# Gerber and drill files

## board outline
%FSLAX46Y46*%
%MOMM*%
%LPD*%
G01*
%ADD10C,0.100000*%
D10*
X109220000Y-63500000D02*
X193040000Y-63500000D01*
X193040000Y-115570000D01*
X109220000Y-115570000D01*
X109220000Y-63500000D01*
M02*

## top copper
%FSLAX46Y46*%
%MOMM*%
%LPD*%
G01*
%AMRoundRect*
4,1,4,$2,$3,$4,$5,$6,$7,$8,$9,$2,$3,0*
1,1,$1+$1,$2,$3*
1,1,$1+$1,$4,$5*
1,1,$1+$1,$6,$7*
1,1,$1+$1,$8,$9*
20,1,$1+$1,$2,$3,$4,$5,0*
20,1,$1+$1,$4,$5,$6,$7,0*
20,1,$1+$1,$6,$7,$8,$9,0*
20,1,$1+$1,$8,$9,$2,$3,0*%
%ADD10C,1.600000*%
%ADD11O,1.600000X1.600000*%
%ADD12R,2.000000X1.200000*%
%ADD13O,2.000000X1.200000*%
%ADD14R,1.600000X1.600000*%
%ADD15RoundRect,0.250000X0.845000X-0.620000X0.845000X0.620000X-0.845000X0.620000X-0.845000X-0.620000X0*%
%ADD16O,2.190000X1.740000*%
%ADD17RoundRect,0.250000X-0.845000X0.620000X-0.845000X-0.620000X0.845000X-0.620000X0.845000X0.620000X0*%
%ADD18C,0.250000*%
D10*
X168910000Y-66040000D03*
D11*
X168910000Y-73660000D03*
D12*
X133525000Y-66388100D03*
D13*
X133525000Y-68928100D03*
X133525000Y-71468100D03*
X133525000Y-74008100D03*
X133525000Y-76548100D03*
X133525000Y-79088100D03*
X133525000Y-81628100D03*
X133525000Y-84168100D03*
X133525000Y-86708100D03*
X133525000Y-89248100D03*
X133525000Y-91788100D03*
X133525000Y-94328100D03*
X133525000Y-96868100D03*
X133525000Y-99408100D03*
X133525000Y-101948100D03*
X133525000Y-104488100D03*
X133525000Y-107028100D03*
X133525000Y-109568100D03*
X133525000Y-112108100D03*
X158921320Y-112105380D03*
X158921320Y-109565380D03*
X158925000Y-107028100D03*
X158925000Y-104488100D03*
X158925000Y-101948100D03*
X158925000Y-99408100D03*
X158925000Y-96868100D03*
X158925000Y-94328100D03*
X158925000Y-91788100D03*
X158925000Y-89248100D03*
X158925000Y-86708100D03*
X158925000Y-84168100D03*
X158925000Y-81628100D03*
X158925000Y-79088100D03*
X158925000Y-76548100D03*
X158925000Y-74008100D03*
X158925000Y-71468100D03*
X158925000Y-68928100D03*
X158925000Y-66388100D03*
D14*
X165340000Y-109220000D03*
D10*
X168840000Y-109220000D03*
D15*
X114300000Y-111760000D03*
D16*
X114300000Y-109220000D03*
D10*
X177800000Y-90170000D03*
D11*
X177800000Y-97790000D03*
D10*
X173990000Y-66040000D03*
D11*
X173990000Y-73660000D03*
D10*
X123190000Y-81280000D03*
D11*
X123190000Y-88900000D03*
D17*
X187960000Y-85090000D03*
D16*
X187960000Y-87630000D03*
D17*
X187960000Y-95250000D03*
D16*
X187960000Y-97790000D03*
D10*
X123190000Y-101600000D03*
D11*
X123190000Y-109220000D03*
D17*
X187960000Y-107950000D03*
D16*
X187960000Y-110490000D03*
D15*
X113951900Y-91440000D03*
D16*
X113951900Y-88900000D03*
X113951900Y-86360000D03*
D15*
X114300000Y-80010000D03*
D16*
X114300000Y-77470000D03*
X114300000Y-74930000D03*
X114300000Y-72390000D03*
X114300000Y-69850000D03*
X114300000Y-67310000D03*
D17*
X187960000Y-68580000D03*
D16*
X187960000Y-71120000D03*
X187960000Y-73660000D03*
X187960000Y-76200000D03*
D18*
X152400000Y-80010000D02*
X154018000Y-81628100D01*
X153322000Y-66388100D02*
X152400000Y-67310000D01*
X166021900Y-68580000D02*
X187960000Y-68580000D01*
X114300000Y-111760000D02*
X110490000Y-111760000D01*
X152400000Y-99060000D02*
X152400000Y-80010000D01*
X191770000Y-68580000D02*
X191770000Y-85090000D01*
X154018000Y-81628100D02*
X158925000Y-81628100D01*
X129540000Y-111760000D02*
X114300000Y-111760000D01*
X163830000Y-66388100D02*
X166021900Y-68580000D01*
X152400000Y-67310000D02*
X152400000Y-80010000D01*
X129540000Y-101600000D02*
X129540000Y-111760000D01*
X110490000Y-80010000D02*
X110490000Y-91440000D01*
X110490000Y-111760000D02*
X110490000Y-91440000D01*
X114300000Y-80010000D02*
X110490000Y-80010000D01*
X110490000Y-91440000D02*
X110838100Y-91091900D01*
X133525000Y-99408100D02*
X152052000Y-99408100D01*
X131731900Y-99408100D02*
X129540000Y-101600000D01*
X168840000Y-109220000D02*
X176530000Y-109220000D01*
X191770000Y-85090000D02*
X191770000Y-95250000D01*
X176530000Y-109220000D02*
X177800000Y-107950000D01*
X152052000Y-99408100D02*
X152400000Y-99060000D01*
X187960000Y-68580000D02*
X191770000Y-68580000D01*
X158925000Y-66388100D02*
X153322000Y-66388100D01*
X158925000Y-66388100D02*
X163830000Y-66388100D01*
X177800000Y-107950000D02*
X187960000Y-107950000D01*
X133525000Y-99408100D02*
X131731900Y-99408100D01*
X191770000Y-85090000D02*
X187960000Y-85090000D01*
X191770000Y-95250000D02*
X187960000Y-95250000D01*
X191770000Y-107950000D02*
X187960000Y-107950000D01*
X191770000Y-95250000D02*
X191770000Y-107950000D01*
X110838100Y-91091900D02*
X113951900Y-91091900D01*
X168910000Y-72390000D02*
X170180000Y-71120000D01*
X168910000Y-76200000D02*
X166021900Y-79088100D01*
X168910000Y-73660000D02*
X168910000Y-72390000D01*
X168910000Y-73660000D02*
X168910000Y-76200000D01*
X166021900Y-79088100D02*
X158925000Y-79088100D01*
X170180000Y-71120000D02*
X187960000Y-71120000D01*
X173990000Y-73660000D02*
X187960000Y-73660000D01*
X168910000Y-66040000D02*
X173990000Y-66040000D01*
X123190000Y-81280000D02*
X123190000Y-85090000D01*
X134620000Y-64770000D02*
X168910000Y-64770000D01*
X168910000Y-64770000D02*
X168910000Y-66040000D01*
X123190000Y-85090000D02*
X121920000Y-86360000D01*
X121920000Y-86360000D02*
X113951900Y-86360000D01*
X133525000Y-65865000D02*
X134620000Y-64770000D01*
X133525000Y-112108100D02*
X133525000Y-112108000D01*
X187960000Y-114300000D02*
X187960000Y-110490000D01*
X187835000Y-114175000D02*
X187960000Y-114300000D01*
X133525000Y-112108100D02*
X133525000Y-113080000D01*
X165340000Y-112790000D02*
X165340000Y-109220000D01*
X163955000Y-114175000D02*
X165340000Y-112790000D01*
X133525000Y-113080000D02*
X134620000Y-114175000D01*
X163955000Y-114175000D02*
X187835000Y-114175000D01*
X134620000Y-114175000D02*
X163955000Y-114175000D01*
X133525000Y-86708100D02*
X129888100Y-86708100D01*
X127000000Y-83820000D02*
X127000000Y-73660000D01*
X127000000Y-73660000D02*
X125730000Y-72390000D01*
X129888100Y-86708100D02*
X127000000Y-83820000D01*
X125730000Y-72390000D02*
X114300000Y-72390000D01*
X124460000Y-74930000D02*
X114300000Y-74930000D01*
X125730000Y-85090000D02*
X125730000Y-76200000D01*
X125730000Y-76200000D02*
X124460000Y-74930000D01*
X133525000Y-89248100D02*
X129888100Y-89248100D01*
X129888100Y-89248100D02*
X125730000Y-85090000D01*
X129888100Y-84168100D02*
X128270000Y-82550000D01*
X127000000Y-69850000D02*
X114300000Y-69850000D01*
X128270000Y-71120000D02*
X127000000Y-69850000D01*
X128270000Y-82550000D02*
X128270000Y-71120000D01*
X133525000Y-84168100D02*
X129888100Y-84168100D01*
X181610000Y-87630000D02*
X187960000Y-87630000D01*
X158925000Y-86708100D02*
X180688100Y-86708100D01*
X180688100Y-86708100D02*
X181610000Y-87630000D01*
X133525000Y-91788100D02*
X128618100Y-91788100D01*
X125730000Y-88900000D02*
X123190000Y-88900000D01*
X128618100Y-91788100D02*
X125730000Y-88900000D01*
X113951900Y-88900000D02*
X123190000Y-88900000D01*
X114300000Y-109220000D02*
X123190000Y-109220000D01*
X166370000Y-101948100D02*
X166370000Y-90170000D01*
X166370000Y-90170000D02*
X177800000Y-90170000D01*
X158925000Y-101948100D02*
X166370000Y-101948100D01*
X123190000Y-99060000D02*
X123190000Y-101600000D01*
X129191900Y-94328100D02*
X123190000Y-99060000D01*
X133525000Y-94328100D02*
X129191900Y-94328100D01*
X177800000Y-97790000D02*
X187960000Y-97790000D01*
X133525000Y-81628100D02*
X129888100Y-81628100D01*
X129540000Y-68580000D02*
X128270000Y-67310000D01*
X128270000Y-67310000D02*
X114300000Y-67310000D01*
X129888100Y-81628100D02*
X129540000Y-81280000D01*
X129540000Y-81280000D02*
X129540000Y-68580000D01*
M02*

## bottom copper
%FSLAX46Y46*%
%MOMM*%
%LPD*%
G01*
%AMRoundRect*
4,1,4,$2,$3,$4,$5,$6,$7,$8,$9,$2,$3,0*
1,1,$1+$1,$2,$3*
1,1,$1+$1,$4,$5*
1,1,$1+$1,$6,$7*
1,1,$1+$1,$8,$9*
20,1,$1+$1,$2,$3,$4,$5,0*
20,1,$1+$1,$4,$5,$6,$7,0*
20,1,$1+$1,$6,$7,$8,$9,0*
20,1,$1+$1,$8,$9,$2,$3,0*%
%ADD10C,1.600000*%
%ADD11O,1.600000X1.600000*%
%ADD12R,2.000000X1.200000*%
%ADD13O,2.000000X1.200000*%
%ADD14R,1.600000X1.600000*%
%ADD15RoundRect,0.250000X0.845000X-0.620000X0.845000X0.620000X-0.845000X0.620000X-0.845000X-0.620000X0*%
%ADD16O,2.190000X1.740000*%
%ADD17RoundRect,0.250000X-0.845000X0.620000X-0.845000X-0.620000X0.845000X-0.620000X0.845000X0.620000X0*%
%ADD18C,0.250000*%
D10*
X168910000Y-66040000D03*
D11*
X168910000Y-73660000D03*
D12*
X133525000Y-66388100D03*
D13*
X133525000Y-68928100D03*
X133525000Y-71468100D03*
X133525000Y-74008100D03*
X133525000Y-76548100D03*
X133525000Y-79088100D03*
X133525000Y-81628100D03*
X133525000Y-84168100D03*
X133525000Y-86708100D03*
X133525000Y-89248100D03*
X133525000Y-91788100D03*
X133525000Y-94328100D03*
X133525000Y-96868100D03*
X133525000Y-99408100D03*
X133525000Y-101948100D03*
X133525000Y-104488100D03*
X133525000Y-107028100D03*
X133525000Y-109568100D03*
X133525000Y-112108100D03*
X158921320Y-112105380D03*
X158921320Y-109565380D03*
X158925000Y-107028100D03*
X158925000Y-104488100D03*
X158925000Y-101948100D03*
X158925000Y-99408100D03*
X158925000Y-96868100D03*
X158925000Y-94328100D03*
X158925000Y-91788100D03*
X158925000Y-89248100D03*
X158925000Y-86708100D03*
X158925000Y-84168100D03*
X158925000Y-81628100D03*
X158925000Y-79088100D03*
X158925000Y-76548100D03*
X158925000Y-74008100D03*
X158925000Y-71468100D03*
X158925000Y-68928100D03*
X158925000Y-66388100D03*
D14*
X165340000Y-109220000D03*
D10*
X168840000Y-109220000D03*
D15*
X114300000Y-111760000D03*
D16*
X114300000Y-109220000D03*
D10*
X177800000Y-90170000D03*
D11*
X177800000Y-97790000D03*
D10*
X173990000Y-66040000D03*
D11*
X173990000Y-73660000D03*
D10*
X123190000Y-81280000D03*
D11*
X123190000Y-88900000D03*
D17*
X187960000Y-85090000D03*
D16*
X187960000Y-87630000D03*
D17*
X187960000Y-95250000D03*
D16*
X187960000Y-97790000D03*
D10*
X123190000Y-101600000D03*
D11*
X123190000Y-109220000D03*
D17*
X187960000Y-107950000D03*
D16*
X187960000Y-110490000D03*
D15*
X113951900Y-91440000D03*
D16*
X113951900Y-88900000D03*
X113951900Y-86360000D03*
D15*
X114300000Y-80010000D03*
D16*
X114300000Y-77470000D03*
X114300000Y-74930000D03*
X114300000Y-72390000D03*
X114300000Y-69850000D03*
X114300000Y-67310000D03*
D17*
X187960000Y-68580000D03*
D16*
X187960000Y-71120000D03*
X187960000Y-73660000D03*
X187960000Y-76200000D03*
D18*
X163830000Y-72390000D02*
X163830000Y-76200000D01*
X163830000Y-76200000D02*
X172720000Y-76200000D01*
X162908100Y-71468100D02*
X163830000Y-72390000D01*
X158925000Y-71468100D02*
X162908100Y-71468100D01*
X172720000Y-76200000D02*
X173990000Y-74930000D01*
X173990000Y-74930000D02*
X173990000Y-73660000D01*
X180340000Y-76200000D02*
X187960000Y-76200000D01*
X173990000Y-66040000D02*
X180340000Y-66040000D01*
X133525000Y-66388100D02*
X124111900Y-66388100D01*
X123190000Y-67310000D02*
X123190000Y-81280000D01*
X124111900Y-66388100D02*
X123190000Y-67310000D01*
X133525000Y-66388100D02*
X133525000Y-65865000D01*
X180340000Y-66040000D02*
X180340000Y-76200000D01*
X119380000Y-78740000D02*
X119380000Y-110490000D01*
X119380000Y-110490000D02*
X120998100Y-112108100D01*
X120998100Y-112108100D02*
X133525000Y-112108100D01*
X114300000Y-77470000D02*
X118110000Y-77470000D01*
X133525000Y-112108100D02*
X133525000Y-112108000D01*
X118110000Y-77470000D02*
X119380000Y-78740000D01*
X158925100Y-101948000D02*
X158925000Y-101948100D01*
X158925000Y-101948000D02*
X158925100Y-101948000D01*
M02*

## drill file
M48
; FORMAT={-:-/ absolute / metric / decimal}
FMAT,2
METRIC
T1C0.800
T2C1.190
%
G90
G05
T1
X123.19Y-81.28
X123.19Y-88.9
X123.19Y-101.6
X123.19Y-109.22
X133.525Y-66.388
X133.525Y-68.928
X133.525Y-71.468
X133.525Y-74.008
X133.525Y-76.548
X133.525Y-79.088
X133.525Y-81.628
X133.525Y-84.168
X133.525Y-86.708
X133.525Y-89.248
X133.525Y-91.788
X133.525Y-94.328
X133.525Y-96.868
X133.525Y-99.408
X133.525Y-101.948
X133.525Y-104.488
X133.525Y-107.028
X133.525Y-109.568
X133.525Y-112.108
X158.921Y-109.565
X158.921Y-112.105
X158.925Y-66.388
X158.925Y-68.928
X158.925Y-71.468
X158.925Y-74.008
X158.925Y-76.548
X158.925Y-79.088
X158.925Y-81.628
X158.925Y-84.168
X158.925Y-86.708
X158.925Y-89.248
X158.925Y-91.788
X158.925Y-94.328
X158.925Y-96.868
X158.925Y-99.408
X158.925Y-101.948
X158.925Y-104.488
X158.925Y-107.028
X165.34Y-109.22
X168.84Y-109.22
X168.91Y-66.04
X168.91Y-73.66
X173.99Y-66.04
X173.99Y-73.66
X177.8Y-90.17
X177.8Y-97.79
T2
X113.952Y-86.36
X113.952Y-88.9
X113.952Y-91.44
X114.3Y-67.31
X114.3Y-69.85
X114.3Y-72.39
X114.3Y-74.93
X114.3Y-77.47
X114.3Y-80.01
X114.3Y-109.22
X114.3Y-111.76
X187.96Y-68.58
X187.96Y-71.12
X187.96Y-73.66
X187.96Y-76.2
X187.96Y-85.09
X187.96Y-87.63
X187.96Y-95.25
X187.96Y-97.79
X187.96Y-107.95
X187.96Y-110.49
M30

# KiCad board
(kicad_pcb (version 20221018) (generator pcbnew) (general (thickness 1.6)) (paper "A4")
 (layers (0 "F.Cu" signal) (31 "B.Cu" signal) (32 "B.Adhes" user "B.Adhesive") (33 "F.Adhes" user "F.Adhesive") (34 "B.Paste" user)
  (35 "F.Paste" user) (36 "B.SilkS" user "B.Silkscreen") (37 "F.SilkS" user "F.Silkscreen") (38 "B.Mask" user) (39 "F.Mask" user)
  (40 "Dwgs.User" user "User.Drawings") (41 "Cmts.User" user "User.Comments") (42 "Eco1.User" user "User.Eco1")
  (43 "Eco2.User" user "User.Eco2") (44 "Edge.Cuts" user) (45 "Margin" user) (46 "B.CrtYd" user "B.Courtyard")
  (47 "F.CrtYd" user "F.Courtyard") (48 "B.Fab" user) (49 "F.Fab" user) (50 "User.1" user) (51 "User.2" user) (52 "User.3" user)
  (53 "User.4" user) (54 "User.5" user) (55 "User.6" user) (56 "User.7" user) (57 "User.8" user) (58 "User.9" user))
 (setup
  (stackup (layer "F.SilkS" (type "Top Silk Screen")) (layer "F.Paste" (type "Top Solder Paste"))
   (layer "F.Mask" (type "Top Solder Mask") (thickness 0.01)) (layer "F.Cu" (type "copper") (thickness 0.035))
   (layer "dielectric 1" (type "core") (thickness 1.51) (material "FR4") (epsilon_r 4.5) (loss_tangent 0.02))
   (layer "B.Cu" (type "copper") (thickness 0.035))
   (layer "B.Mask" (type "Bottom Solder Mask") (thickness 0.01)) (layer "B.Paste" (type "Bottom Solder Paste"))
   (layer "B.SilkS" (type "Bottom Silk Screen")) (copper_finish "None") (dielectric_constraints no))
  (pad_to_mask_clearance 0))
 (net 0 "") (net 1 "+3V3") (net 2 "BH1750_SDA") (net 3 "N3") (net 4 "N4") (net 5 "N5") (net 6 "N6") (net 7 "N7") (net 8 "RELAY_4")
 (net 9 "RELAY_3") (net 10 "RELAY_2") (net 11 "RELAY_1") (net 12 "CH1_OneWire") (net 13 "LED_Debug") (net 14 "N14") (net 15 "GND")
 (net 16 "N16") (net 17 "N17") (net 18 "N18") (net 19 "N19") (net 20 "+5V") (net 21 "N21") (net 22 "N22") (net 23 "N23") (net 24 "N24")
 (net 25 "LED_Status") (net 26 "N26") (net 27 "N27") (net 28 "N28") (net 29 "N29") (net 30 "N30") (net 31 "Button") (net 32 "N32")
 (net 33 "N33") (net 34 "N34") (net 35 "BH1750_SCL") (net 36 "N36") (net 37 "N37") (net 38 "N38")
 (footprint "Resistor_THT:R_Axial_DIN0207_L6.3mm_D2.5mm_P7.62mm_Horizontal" (layer "F.Cu") (at 168.91 66.04 -90)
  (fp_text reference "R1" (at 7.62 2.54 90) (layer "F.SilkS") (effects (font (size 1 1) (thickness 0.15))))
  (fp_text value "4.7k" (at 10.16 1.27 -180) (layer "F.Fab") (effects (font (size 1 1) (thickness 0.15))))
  (pad "1" thru_hole circle (at 0 0 270) (size 1.6 1.6) (drill 0.8) (layers "*.Cu" "*.Mask") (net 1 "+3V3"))
  (pad "2" thru_hole oval (at 7.62 0 270) (size 1.6 1.6) (drill 0.8) (layers "*.Cu" "*.Mask") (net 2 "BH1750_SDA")))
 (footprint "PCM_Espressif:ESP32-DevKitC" (layer "F.Cu") (at 133.525 66.3881)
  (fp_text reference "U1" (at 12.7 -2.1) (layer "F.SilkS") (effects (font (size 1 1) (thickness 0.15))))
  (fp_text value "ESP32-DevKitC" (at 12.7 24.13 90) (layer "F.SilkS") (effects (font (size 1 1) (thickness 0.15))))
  (pad "1" thru_hole rect (at 0 0 270) (size 1.2 2) (drill 0.8) (layers "*.Cu" "*.Mask") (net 1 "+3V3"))
  (pad "2" thru_hole oval (at 0 2.54 270) (size 1.2 2) (drill 0.8) (layers "*.Cu" "*.Mask") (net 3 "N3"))
  (pad "3" thru_hole oval (at 0 5.08 270) (size 1.2 2) (drill 0.8) (layers "*.Cu" "*.Mask") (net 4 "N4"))
  (pad "4" thru_hole oval (at 0 7.62 270) (size 1.2 2) (drill 0.8) (layers "*.Cu" "*.Mask") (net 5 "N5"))
  (pad "5" thru_hole oval (at 0 10.16 270) (size 1.2 2) (drill 0.8) (layers "*.Cu" "*.Mask") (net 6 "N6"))
  (pad "6" thru_hole oval (at 0 12.7 270) (size 1.2 2) (drill 0.8) (layers "*.Cu" "*.Mask") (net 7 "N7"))
  (pad "7" thru_hole oval (at 0 15.24 270) (size 1.2 2) (drill 0.8) (layers "*.Cu" "*.Mask") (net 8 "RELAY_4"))
  (pad "8" thru_hole oval (at 0 17.78 270) (size 1.2 2) (drill 0.8) (layers "*.Cu" "*.Mask") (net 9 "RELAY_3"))
  (pad "9" thru_hole oval (at 0 20.32 270) (size 1.2 2) (drill 0.8) (layers "*.Cu" "*.Mask") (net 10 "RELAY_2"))
  (pad "10" thru_hole oval (at 0 22.86 270) (size 1.2 2) (drill 0.8) (layers "*.Cu" "*.Mask") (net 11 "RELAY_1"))
  (pad "11" thru_hole oval (at 0 25.4 270) (size 1.2 2) (drill 0.8) (layers "*.Cu" "*.Mask") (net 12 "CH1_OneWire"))
  (pad "12" thru_hole oval (at 0 27.94 270) (size 1.2 2) (drill 0.8) (layers "*.Cu" "*.Mask") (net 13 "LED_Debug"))
  (pad "13" thru_hole oval (at 0 30.48 270) (size 1.2 2) (drill 0.8) (layers "*.Cu" "*.Mask") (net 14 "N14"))
  (pad "14" thru_hole oval (at 0 33.02 270) (size 1.2 2) (drill 0.8) (layers "*.Cu" "*.Mask") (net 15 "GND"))
  (pad "15" thru_hole oval (at 0 35.56 270) (size 1.2 2) (drill 0.8) (layers "*.Cu" "*.Mask") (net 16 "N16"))
  (pad "16" thru_hole oval (at 0 38.1 270) (size 1.2 2) (drill 0.8) (layers "*.Cu" "*.Mask") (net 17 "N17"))
  (pad "17" thru_hole oval (at 0 40.64 270) (size 1.2 2) (drill 0.8) (layers "*.Cu" "*.Mask") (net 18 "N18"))
  (pad "18" thru_hole oval (at 0 43.18 270) (size 1.2 2) (drill 0.8) (layers "*.Cu" "*.Mask") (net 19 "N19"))
  (pad "19" thru_hole oval (at 0 45.72 270) (size 1.2 2) (drill 0.8) (layers "*.Cu" "*.Mask") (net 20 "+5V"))
  (pad "20" thru_hole oval (at 25.39632 45.71728 270) (size 1.2 2) (drill 0.8) (layers "*.Cu" "*.Mask") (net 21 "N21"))
  (pad "21" thru_hole oval (at 25.39632 43.17728 270) (size 1.2 2) (drill 0.8) (layers "*.Cu" "*.Mask") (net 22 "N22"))
  (pad "22" thru_hole oval (at 25.4 40.64 270) (size 1.2 2) (drill 0.8) (layers "*.Cu" "*.Mask") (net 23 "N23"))
  (pad "23" thru_hole oval (at 25.4 38.1 270) (size 1.2 2) (drill 0.8) (layers "*.Cu" "*.Mask") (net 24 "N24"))
  (pad "24" thru_hole oval (at 25.4 35.56 270) (size 1.2 2) (drill 0.8) (layers "*.Cu" "*.Mask") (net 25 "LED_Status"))
  (pad "25" thru_hole oval (at 25.4 33.02 270) (size 1.2 2) (drill 0.8) (layers "*.Cu" "*.Mask") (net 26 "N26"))
  (pad "26" thru_hole oval (at 25.4 30.48 270) (size 1.2 2) (drill 0.8) (layers "*.Cu" "*.Mask") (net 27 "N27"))
  (pad "27" thru_hole oval (at 25.4 27.94 270) (size 1.2 2) (drill 0.8) (layers "*.Cu" "*.Mask") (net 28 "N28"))
  (pad "28" thru_hole oval (at 25.4 25.4 270) (size 1.2 2) (drill 0.8) (layers "*.Cu" "*.Mask") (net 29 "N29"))
  (pad "29" thru_hole oval (at 25.4 22.86 270) (size 1.2 2) (drill 0.8) (layers "*.Cu" "*.Mask") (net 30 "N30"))
  (pad "30" thru_hole oval (at 25.4 20.32 270) (size 1.2 2) (drill 0.8) (layers "*.Cu" "*.Mask") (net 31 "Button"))
  (pad "31" thru_hole oval (at 25.4 17.78 270) (size 1.2 2) (drill 0.8) (layers "*.Cu" "*.Mask") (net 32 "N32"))
  (pad "32" thru_hole oval (at 25.4 15.24 270) (size 1.2 2) (drill 0.8) (layers "*.Cu" "*.Mask") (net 15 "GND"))
  (pad "33" thru_hole oval (at 25.4 12.7 270) (size 1.2 2) (drill 0.8) (layers "*.Cu" "*.Mask") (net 2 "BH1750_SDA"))
  (pad "34" thru_hole oval (at 25.4 10.16 270) (size 1.2 2) (drill 0.8) (layers "*.Cu" "*.Mask") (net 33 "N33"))
  (pad "35" thru_hole oval (at 25.4 7.62 270) (size 1.2 2) (drill 0.8) (layers "*.Cu" "*.Mask") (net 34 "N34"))
  (pad "36" thru_hole oval (at 25.4 5.08 270) (size 1.2 2) (drill 0.8) (layers "*.Cu" "*.Mask") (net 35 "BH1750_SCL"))
  (pad "37" thru_hole oval (at 25.4 2.54 270) (size 1.2 2) (drill 0.8) (layers "*.Cu" "*.Mask") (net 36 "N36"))
  (pad "38" thru_hole oval (at 25.4 0 270) (size 1.2 2) (drill 0.8) (layers "*.Cu" "*.Mask") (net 15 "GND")))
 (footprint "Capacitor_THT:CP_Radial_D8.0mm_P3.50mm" (layer "F.Cu") (at 165.34 109.22)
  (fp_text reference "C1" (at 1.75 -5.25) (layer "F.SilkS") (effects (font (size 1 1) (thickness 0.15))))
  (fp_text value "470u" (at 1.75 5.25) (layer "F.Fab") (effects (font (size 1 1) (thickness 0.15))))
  (pad "1" thru_hole rect (at 0 0) (size 1.6 1.6) (drill 0.8) (layers "*.Cu" "*.Mask") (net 20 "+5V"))
  (pad "2" thru_hole circle (at 3.5 0) (size 1.6 1.6) (drill 0.8) (layers "*.Cu" "*.Mask") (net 15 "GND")))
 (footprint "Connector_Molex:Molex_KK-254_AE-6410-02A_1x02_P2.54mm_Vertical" (layer "F.Cu") (at 114.3 111.76 90)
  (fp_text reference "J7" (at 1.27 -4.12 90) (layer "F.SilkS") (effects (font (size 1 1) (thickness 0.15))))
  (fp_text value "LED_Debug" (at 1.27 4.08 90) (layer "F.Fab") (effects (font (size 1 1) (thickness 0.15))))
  (pad "1" thru_hole roundrect (at 0 0 90) (size 1.74 2.19) (drill 1.19) (layers "*.Cu" "*.Mask") (roundrect_rratio 0.143678) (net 15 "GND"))
  (pad "2" thru_hole oval (at 2.54 0 90) (size 1.74 2.19) (drill 1.19) (layers "*.Cu" "*.Mask") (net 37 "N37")))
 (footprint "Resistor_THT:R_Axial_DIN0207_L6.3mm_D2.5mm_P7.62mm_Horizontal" (layer "F.Cu") (at 177.8 90.17 -90)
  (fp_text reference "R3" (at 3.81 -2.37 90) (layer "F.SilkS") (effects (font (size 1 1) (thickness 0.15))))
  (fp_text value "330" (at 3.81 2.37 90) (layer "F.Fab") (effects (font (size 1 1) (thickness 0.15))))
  (pad "1" thru_hole circle (at 0 0 270) (size 1.6 1.6) (drill 0.8) (layers "*.Cu" "*.Mask") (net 25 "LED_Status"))
  (pad "2" thru_hole oval (at 7.62 0 270) (size 1.6 1.6) (drill 0.8) (layers "*.Cu" "*.Mask") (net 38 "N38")))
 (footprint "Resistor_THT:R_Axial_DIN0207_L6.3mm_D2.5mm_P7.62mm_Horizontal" (layer "F.Cu") (at 173.99 66.04 -90)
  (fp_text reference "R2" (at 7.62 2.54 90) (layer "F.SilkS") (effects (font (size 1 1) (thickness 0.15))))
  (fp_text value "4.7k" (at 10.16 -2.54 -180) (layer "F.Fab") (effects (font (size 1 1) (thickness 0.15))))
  (pad "1" thru_hole circle (at 0 0 270) (size 1.6 1.6) (drill 0.8) (layers "*.Cu" "*.Mask") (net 1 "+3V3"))
  (pad "2" thru_hole oval (at 7.62 0 270) (size 1.6 1.6) (drill 0.8) (layers "*.Cu" "*.Mask") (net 35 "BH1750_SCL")))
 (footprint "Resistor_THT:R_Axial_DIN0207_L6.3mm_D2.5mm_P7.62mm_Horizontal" (layer "F.Cu") (at 123.19 81.28 -90)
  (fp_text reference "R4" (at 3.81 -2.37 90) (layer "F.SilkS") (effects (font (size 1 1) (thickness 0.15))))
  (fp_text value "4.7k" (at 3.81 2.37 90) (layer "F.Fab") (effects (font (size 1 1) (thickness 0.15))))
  (pad "1" thru_hole circle (at 0 0 270) (size 1.6 1.6) (drill 0.8) (layers "*.Cu" "*.Mask") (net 1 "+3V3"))
  (pad "2" thru_hole oval (at 7.62 0 270) (size 1.6 1.6) (drill 0.8) (layers "*.Cu" "*.Mask") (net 12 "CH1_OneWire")))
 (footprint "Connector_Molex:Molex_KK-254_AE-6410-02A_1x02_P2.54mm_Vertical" (layer "F.Cu") (at 187.96 85.09 -90)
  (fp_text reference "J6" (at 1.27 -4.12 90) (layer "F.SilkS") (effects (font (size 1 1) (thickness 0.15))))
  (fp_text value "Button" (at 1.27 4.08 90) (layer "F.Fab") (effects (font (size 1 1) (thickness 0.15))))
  (pad "1" thru_hole roundrect (at 0 0 270) (size 1.74 2.19) (drill 1.19) (layers "*.Cu" "*.Mask") (roundrect_rratio 0.1436781609)
   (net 15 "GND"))
  (pad "2" thru_hole oval (at 2.54 0 270) (size 1.74 2.19) (drill 1.19) (layers "*.Cu" "*.Mask") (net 31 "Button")))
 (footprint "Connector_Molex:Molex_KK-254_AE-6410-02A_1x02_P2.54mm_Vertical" (layer "F.Cu") (at 187.96 95.25 -90)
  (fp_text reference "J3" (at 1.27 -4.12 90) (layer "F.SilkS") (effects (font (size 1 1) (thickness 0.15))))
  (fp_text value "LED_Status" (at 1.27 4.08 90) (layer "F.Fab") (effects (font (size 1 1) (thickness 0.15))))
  (pad "1" thru_hole roundrect (at 0 0 270) (size 1.74 2.19) (drill 1.19) (layers "*.Cu" "*.Mask") (roundrect_rratio 0.1436781609)
   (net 15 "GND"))
  (pad "2" thru_hole oval (at 2.54 0 270) (size 1.74 2.19) (drill 1.19) (layers "*.Cu" "*.Mask") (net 38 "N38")))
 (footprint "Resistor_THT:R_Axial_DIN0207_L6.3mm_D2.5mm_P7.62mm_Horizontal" (layer "F.Cu") (at 123.19 101.6 -90)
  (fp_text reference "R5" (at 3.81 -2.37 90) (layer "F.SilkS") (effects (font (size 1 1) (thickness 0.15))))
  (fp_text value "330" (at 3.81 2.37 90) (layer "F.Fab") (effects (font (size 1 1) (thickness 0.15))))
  (pad "1" thru_hole circle (at 0 0 270) (size 1.6 1.6) (drill 0.8) (layers "*.Cu" "*.Mask") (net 13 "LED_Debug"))
  (pad "2" thru_hole oval (at 7.62 0 270) (size 1.6 1.6) (drill 0.8) (layers "*.Cu" "*.Mask") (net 37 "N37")))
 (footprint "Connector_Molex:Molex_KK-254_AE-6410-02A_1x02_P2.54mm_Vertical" (layer "F.Cu") (at 187.96 107.95 -90)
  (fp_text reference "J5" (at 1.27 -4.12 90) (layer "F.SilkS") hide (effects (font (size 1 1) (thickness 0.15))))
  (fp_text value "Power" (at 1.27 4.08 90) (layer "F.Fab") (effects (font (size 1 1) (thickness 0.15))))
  (pad "1" thru_hole roundrect (at 0 0 270) (size 1.74 2.19) (drill 1.19) (layers "*.Cu" "*.Mask") (roundrect_rratio 0.1436781609)
   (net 15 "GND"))
  (pad "2" thru_hole oval (at 2.54 0 270) (size 1.74 2.19) (drill 1.19) (layers "*.Cu" "*.Mask") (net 20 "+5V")))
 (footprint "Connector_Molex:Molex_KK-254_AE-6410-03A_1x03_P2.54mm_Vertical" (layer "F.Cu") (at 113.9519 91.44 90)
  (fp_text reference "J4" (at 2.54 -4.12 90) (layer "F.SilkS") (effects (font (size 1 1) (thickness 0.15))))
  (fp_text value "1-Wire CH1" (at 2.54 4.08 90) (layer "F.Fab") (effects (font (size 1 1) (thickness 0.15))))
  (pad "1" thru_hole roundrect (at 0 0 90) (size 1.74 2.19) (drill 1.19) (layers "*.Cu" "*.Mask") (roundrect_rratio 0.1436781609)
   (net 15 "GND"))
  (pad "2" thru_hole oval (at 2.54 0 90) (size 1.74 2.19) (drill 1.19) (layers "*.Cu" "*.Mask") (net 12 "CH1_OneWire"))
  (pad "3" thru_hole oval (at 5.08 0 90) (size 1.74 2.19) (drill 1.19) (layers "*.Cu" "*.Mask") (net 1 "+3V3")))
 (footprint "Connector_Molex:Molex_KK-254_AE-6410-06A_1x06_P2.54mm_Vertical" (layer "F.Cu") (at 114.3 80.01 90)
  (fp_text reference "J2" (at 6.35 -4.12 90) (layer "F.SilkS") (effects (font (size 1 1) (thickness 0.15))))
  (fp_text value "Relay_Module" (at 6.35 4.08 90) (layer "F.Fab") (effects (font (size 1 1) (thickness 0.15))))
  (pad "1" thru_hole roundrect (at 0 0 90) (size 1.74 2.19) (drill 1.19) (layers "*.Cu" "*.Mask") (roundrect_rratio 0.1436781609)
   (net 15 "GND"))
  (pad "2" thru_hole oval (at 2.54 0 90) (size 1.74 2.19) (drill 1.19) (layers "*.Cu" "*.Mask") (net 20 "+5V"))
  (pad "3" thru_hole oval (at 5.08 0 90) (size 1.74 2.19) (drill 1.19) (layers "*.Cu" "*.Mask") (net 11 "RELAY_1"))
  (pad "4" thru_hole oval (at 7.62 0 90) (size 1.74 2.19) (drill 1.19) (layers "*.Cu" "*.Mask") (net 10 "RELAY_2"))
  (pad "5" thru_hole oval (at 10.16 0 90) (size 1.74 2.19) (drill 1.19) (layers "*.Cu" "*.Mask") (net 9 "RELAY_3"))
  (pad "6" thru_hole oval (at 12.7 0 90) (size 1.74 2.19) (drill 1.19) (layers "*.Cu" "*.Mask") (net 8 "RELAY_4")))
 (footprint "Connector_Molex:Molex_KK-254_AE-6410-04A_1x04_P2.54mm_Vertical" (layer "F.Cu") (at 187.96 68.58 -90)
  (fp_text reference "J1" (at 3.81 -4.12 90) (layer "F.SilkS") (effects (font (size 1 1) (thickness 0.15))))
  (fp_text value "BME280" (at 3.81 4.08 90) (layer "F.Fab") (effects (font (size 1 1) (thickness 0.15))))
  (pad "1" thru_hole roundrect (at 0 0 270) (size 1.74 2.19) (drill 1.19) (layers "*.Cu" "*.Mask") (roundrect_rratio 0.1436781609)
   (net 15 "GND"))
  (pad "2" thru_hole oval (at 2.54 0 270) (size 1.74 2.19) (drill 1.19) (layers "*.Cu" "*.Mask") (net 2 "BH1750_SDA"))
  (pad "3" thru_hole oval (at 5.08 0 270) (size 1.74 2.19) (drill 1.19) (layers "*.Cu" "*.Mask") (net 35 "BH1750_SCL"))
  (pad "4" thru_hole oval (at 7.62 0 270) (size 1.74 2.19) (drill 1.19) (layers "*.Cu" "*.Mask") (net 1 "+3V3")))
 (gr_rect (start 109.22 63.5) (end 193.04 115.57) (stroke (width 0.1) (type default)) (fill none) (layer "Edge.Cuts"))
 (segment (start 152.4 80.01) (end 154.018 81.6281) (width 0.25) (layer "F.Cu") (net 15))
 (segment (start 153.322 66.3881) (end 152.4 67.31) (width 0.25) (layer "F.Cu") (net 15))
 (segment (start 166.0219 68.58) (end 187.96 68.58) (width 0.25) (layer "F.Cu") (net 15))
 (segment (start 114.3 111.76) (end 110.49 111.76) (width 0.25) (layer "F.Cu") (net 15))
 (segment (start 152.4 99.06) (end 152.4 80.01) (width 0.25) (layer "F.Cu") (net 15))
 (segment (start 191.77 68.58) (end 191.77 85.09) (width 0.25) (layer "F.Cu") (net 15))
 (segment (start 154.018 81.6281) (end 158.925 81.6281) (width 0.25) (layer "F.Cu") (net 15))
 (segment (start 129.54 111.76) (end 114.3 111.76) (width 0.25) (layer "F.Cu") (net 15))
 (segment (start 163.83 66.3881) (end 166.0219 68.58) (width 0.25) (layer "F.Cu") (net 15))
 (segment (start 152.4 67.31) (end 152.4 80.01) (width 0.25) (layer "F.Cu") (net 15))
 (segment (start 129.54 101.6) (end 129.54 111.76) (width 0.25) (layer "F.Cu") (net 15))
 (segment (start 110.49 80.01) (end 110.49 91.44) (width 0.25) (layer "F.Cu") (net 15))
 (segment (start 110.49 111.76) (end 110.49 91.44) (width 0.25) (layer "F.Cu") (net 15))
 (segment (start 114.3 80.01) (end 110.49 80.01) (width 0.25) (layer "F.Cu") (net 15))
 (segment (start 110.49 91.44) (end 110.8381 91.0919) (width 0.25) (layer "F.Cu") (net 15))
 (segment (start 133.525 99.4081) (end 152.052 99.4081) (width 0.25) (layer "F.Cu") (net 15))
 (segment (start 131.7319 99.4081) (end 129.54 101.6) (width 0.25) (layer "F.Cu") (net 15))
 (segment (start 168.84 109.22) (end 176.53 109.22) (width 0.25) (layer "F.Cu") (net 15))
 (segment (start 191.77 85.09) (end 191.77 95.25) (width 0.25) (layer "F.Cu") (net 15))
 (segment (start 176.53 109.22) (end 177.8 107.95) (width 0.25) (layer "F.Cu") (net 15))
 (segment (start 152.052 99.4081) (end 152.4 99.06) (width 0.25) (layer "F.Cu") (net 15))
 (segment (start 187.96 68.58) (end 191.77 68.58) (width 0.25) (layer "F.Cu") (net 15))
 (segment (start 158.925 66.3881) (end 153.322 66.3881) (width 0.25) (layer "F.Cu") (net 15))
 (segment (start 158.925 66.3881) (end 163.83 66.3881) (width 0.25) (layer "F.Cu") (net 15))
 (segment (start 177.8 107.95) (end 187.96 107.95) (width 0.25) (layer "F.Cu") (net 15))
 (segment (start 133.525 99.4081) (end 131.7319 99.4081) (width 0.25) (layer "F.Cu") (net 15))
 (segment (start 191.77 85.09) (end 187.96 85.09) (width 0.25) (layer "F.Cu") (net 15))
 (segment (start 191.77 95.25) (end 187.96 95.25) (width 0.25) (layer "F.Cu") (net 15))
 (segment (start 191.77 107.95) (end 187.96 107.95) (width 0.25) (layer "F.Cu") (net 15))
 (segment (start 191.77 95.25) (end 191.77 107.95) (width 0.25) (layer "F.Cu") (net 15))
 (segment (start 110.8381 91.0919) (end 113.9519 91.0919) (width 0.25) (layer "F.Cu") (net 15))
 (segment (start 168.91 72.39) (end 170.18 71.12) (width 0.25) (layer "F.Cu") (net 2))
 (segment (start 168.91 76.2) (end 166.0219 79.0881) (width 0.25) (layer "F.Cu") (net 2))
 (segment (start 168.91 73.66) (end 168.91 72.39) (width 0.25) (layer "F.Cu") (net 2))
 (segment (start 168.91 73.66) (end 168.91 76.2) (width 0.25) (layer "F.Cu") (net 2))
 (segment (start 166.0219 79.0881) (end 158.925 79.0881) (width 0.25) (layer "F.Cu") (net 2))
 (segment (start 170.18 71.12) (end 187.96 71.12) (width 0.25) (layer "F.Cu") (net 2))
 (segment (start 173.99 73.66) (end 187.96 73.66) (width 0.25) (layer "F.Cu") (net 35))
 (segment (start 163.83 72.39) (end 163.83 76.2) (width 0.25) (layer "B.Cu") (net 35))
 (segment (start 163.83 76.2) (end 172.72 76.2) (width 0.25) (layer "B.Cu") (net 35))
 (segment (start 162.9081 71.4681) (end 163.83 72.39) (width 0.25) (layer "B.Cu") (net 35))
 (segment (start 158.925 71.4681) (end 162.9081 71.4681) (width 0.25) (layer "B.Cu") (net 35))
 (segment (start 172.72 76.2) (end 173.99 74.93) (width 0.25) (layer "B.Cu") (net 35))
 (segment (start 173.99 74.93) (end 173.99 73.66) (width 0.25) (layer "B.Cu") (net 35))
 (segment (start 168.91 66.04) (end 173.99 66.04) (width 0.25) (layer "F.Cu") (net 1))
 (segment (start 123.19 81.28) (end 123.19 85.09) (width 0.25) (layer "F.Cu") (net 1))
 (segment (start 134.62 64.77) (end 168.91 64.77) (width 0.25) (layer "F.Cu") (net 1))
 (segment (start 168.91 64.77) (end 168.91 66.04) (width 0.25) (layer "F.Cu") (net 1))
 (segment (start 123.19 85.09) (end 121.92 86.36) (width 0.25) (layer "F.Cu") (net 1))
 (segment (start 121.92 86.36) (end 113.9519 86.36) (width 0.25) (layer "F.Cu") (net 1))
 (segment (start 133.525 65.865) (end 134.62 64.77) (width 0.25) (layer "F.Cu") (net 1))
 (segment (start 180.34 76.2) (end 187.96 76.2) (width 0.25) (layer "B.Cu") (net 1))
 (segment (start 173.99 66.04) (end 180.34 66.04) (width 0.25) (layer "B.Cu") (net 1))
 (segment (start 133.525 66.3881) (end 124.1119 66.3881) (width 0.25) (layer "B.Cu") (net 1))
 (segment (start 123.19 67.31) (end 123.19 81.28) (width 0.25) (layer "B.Cu") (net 1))
 (segment (start 124.1119 66.3881) (end 123.19 67.31) (width 0.25) (layer "B.Cu") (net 1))
 (segment (start 133.525 66.3881) (end 133.525 65.865) (width 0.25) (layer "B.Cu") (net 1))
 (segment (start 180.34 66.04) (end 180.34 76.2) (width 0.25) (layer "B.Cu") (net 1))
 (segment (start 133.525 112.1081) (end 133.525 112.108) (width 0.25) (layer "F.Cu") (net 20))
 (segment (start 187.96 114.3) (end 187.96 110.49) (width 0.25) (layer "F.Cu") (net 20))
 (segment (start 187.835 114.175) (end 187.96 114.3) (width 0.25) (layer "F.Cu") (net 20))
 (segment (start 133.525 112.1081) (end 133.525 113.08) (width 0.25) (layer "F.Cu") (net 20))
 (segment (start 165.34 112.79) (end 165.34 109.22) (width 0.25) (layer "F.Cu") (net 20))
 (segment (start 163.955 114.175) (end 165.34 112.79) (width 0.25) (layer "F.Cu") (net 20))
 (segment (start 133.525 113.08) (end 134.62 114.175) (width 0.25) (layer "F.Cu") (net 20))
 (segment (start 163.955 114.175) (end 187.835 114.175) (width 0.25) (layer "F.Cu") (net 20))
 (segment (start 134.62 114.175) (end 163.955 114.175) (width 0.25) (layer "F.Cu") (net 20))
 (segment (start 119.38 78.74) (end 119.38 110.49) (width 0.25) (layer "B.Cu") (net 20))
 (segment (start 119.38 110.49) (end 120.9981 112.1081) (width 0.25) (layer "B.Cu") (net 20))
 (segment (start 120.9981 112.1081) (end 133.525 112.1081) (width 0.25) (layer "B.Cu") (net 20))
 (segment (start 114.3 77.47) (end 118.11 77.47) (width 0.25) (layer "B.Cu") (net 20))
 (segment (start 133.525 112.1081) (end 133.525 112.108) (width 0.25) (layer "B.Cu") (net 20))
 (segment (start 118.11 77.47) (end 119.38 78.74) (width 0.25) (layer "B.Cu") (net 20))
 (segment (start 133.525 86.7081) (end 129.8881 86.7081) (width 0.25) (layer "F.Cu") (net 10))
 (segment (start 127 83.82) (end 127 73.66) (width 0.25) (layer "F.Cu") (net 10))
 (segment (start 127 73.66) (end 125.73 72.39) (width 0.25) (layer "F.Cu") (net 10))
 (segment (start 129.8881 86.7081) (end 127 83.82) (width 0.25) (layer "F.Cu") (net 10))
 (segment (start 125.73 72.39) (end 114.3 72.39) (width 0.25) (layer "F.Cu") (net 10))
 (segment (start 124.46 74.93) (end 114.3 74.93) (width 0.25) (layer "F.Cu") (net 11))
 (segment (start 125.73 85.09) (end 125.73 76.2) (width 0.25) (layer "F.Cu") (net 11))
 (segment (start 125.73 76.2) (end 124.46 74.93) (width 0.25) (layer "F.Cu") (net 11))
 (segment (start 133.525 89.2481) (end 129.8881 89.2481) (width 0.25) (layer "F.Cu") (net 11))
 (segment (start 129.8881 89.2481) (end 125.73 85.09) (width 0.25) (layer "F.Cu") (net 11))
 (segment (start 129.8881 84.1681) (end 128.27 82.55) (width 0.25) (layer "F.Cu") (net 9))
 (segment (start 127 69.85) (end 114.3 69.85) (width 0.25) (layer "F.Cu") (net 9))
 (segment (start 128.27 71.12) (end 127 69.85) (width 0.25) (layer "F.Cu") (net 9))
 (segment (start 128.27 82.55) (end 128.27 71.12) (width 0.25) (layer "F.Cu") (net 9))
 (segment (start 133.525 84.1681) (end 129.8881 84.1681) (width 0.25) (layer "F.Cu") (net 9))
 (segment (start 181.61 87.63) (end 187.96 87.63) (width 0.25) (layer "F.Cu") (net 31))
 (segment (start 158.925 86.7081) (end 180.6881 86.7081) (width 0.25) (layer "F.Cu") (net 31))
 (segment (start 180.6881 86.7081) (end 181.61 87.63) (width 0.25) (layer "F.Cu") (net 31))
 (segment (start 133.525 91.7881) (end 128.6181 91.7881) (width 0.25) (layer "F.Cu") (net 12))
 (segment (start 125.73 88.9) (end 123.19 88.9) (width 0.25) (layer "F.Cu") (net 12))
 (segment (start 128.6181 91.7881) (end 125.73 88.9) (width 0.25) (layer "F.Cu") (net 12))
 (segment (start 113.9519 88.9) (end 123.19 88.9) (width 0.25) (layer "F.Cu") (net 12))
 (segment (start 114.3 109.22) (end 123.19 109.22) (width 0.25) (layer "F.Cu") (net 37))
 (segment (start 166.37 101.9481) (end 166.37 90.17) (width 0.25) (layer "F.Cu") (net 25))
 (segment (start 166.37 90.17) (end 177.8 90.17) (width 0.25) (layer "F.Cu") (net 25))
 (segment (start 158.925 101.9481) (end 166.37 101.9481) (width 0.25) (layer "F.Cu") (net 25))
 (segment (start 158.9251 101.948) (end 158.925 101.9481) (width 0.25) (layer "B.Cu") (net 25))
 (segment (start 158.925 101.948) (end 158.9251 101.948) (width 0.25) (layer "B.Cu") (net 25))
 (segment (start 123.19 99.06) (end 123.19 101.6) (width 0.25) (layer "F.Cu") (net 13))
 (segment (start 129.1919 94.3281) (end 123.19 99.06) (width 0.25) (layer "F.Cu") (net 13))
 (segment (start 133.525 94.3281) (end 129.1919 94.3281) (width 0.25) (layer "F.Cu") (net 13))
 (segment (start 177.8 97.79) (end 187.96 97.79) (width 0.25) (layer "F.Cu") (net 38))
 (segment (start 133.525 81.6281) (end 129.8881 81.6281) (width 0.25) (layer "F.Cu") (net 8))
 (segment (start 129.54 68.58) (end 128.27 67.31) (width 0.25) (layer "F.Cu") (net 8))
 (segment (start 128.27 67.31) (end 114.3 67.31) (width 0.25) (layer "F.Cu") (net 8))
 (segment (start 129.8881 81.6281) (end 129.54 81.28) (width 0.25) (layer "F.Cu") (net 8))
 (segment (start 129.54 81.28) (end 129.54 68.58) (width 0.25) (layer "F.Cu") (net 8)))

